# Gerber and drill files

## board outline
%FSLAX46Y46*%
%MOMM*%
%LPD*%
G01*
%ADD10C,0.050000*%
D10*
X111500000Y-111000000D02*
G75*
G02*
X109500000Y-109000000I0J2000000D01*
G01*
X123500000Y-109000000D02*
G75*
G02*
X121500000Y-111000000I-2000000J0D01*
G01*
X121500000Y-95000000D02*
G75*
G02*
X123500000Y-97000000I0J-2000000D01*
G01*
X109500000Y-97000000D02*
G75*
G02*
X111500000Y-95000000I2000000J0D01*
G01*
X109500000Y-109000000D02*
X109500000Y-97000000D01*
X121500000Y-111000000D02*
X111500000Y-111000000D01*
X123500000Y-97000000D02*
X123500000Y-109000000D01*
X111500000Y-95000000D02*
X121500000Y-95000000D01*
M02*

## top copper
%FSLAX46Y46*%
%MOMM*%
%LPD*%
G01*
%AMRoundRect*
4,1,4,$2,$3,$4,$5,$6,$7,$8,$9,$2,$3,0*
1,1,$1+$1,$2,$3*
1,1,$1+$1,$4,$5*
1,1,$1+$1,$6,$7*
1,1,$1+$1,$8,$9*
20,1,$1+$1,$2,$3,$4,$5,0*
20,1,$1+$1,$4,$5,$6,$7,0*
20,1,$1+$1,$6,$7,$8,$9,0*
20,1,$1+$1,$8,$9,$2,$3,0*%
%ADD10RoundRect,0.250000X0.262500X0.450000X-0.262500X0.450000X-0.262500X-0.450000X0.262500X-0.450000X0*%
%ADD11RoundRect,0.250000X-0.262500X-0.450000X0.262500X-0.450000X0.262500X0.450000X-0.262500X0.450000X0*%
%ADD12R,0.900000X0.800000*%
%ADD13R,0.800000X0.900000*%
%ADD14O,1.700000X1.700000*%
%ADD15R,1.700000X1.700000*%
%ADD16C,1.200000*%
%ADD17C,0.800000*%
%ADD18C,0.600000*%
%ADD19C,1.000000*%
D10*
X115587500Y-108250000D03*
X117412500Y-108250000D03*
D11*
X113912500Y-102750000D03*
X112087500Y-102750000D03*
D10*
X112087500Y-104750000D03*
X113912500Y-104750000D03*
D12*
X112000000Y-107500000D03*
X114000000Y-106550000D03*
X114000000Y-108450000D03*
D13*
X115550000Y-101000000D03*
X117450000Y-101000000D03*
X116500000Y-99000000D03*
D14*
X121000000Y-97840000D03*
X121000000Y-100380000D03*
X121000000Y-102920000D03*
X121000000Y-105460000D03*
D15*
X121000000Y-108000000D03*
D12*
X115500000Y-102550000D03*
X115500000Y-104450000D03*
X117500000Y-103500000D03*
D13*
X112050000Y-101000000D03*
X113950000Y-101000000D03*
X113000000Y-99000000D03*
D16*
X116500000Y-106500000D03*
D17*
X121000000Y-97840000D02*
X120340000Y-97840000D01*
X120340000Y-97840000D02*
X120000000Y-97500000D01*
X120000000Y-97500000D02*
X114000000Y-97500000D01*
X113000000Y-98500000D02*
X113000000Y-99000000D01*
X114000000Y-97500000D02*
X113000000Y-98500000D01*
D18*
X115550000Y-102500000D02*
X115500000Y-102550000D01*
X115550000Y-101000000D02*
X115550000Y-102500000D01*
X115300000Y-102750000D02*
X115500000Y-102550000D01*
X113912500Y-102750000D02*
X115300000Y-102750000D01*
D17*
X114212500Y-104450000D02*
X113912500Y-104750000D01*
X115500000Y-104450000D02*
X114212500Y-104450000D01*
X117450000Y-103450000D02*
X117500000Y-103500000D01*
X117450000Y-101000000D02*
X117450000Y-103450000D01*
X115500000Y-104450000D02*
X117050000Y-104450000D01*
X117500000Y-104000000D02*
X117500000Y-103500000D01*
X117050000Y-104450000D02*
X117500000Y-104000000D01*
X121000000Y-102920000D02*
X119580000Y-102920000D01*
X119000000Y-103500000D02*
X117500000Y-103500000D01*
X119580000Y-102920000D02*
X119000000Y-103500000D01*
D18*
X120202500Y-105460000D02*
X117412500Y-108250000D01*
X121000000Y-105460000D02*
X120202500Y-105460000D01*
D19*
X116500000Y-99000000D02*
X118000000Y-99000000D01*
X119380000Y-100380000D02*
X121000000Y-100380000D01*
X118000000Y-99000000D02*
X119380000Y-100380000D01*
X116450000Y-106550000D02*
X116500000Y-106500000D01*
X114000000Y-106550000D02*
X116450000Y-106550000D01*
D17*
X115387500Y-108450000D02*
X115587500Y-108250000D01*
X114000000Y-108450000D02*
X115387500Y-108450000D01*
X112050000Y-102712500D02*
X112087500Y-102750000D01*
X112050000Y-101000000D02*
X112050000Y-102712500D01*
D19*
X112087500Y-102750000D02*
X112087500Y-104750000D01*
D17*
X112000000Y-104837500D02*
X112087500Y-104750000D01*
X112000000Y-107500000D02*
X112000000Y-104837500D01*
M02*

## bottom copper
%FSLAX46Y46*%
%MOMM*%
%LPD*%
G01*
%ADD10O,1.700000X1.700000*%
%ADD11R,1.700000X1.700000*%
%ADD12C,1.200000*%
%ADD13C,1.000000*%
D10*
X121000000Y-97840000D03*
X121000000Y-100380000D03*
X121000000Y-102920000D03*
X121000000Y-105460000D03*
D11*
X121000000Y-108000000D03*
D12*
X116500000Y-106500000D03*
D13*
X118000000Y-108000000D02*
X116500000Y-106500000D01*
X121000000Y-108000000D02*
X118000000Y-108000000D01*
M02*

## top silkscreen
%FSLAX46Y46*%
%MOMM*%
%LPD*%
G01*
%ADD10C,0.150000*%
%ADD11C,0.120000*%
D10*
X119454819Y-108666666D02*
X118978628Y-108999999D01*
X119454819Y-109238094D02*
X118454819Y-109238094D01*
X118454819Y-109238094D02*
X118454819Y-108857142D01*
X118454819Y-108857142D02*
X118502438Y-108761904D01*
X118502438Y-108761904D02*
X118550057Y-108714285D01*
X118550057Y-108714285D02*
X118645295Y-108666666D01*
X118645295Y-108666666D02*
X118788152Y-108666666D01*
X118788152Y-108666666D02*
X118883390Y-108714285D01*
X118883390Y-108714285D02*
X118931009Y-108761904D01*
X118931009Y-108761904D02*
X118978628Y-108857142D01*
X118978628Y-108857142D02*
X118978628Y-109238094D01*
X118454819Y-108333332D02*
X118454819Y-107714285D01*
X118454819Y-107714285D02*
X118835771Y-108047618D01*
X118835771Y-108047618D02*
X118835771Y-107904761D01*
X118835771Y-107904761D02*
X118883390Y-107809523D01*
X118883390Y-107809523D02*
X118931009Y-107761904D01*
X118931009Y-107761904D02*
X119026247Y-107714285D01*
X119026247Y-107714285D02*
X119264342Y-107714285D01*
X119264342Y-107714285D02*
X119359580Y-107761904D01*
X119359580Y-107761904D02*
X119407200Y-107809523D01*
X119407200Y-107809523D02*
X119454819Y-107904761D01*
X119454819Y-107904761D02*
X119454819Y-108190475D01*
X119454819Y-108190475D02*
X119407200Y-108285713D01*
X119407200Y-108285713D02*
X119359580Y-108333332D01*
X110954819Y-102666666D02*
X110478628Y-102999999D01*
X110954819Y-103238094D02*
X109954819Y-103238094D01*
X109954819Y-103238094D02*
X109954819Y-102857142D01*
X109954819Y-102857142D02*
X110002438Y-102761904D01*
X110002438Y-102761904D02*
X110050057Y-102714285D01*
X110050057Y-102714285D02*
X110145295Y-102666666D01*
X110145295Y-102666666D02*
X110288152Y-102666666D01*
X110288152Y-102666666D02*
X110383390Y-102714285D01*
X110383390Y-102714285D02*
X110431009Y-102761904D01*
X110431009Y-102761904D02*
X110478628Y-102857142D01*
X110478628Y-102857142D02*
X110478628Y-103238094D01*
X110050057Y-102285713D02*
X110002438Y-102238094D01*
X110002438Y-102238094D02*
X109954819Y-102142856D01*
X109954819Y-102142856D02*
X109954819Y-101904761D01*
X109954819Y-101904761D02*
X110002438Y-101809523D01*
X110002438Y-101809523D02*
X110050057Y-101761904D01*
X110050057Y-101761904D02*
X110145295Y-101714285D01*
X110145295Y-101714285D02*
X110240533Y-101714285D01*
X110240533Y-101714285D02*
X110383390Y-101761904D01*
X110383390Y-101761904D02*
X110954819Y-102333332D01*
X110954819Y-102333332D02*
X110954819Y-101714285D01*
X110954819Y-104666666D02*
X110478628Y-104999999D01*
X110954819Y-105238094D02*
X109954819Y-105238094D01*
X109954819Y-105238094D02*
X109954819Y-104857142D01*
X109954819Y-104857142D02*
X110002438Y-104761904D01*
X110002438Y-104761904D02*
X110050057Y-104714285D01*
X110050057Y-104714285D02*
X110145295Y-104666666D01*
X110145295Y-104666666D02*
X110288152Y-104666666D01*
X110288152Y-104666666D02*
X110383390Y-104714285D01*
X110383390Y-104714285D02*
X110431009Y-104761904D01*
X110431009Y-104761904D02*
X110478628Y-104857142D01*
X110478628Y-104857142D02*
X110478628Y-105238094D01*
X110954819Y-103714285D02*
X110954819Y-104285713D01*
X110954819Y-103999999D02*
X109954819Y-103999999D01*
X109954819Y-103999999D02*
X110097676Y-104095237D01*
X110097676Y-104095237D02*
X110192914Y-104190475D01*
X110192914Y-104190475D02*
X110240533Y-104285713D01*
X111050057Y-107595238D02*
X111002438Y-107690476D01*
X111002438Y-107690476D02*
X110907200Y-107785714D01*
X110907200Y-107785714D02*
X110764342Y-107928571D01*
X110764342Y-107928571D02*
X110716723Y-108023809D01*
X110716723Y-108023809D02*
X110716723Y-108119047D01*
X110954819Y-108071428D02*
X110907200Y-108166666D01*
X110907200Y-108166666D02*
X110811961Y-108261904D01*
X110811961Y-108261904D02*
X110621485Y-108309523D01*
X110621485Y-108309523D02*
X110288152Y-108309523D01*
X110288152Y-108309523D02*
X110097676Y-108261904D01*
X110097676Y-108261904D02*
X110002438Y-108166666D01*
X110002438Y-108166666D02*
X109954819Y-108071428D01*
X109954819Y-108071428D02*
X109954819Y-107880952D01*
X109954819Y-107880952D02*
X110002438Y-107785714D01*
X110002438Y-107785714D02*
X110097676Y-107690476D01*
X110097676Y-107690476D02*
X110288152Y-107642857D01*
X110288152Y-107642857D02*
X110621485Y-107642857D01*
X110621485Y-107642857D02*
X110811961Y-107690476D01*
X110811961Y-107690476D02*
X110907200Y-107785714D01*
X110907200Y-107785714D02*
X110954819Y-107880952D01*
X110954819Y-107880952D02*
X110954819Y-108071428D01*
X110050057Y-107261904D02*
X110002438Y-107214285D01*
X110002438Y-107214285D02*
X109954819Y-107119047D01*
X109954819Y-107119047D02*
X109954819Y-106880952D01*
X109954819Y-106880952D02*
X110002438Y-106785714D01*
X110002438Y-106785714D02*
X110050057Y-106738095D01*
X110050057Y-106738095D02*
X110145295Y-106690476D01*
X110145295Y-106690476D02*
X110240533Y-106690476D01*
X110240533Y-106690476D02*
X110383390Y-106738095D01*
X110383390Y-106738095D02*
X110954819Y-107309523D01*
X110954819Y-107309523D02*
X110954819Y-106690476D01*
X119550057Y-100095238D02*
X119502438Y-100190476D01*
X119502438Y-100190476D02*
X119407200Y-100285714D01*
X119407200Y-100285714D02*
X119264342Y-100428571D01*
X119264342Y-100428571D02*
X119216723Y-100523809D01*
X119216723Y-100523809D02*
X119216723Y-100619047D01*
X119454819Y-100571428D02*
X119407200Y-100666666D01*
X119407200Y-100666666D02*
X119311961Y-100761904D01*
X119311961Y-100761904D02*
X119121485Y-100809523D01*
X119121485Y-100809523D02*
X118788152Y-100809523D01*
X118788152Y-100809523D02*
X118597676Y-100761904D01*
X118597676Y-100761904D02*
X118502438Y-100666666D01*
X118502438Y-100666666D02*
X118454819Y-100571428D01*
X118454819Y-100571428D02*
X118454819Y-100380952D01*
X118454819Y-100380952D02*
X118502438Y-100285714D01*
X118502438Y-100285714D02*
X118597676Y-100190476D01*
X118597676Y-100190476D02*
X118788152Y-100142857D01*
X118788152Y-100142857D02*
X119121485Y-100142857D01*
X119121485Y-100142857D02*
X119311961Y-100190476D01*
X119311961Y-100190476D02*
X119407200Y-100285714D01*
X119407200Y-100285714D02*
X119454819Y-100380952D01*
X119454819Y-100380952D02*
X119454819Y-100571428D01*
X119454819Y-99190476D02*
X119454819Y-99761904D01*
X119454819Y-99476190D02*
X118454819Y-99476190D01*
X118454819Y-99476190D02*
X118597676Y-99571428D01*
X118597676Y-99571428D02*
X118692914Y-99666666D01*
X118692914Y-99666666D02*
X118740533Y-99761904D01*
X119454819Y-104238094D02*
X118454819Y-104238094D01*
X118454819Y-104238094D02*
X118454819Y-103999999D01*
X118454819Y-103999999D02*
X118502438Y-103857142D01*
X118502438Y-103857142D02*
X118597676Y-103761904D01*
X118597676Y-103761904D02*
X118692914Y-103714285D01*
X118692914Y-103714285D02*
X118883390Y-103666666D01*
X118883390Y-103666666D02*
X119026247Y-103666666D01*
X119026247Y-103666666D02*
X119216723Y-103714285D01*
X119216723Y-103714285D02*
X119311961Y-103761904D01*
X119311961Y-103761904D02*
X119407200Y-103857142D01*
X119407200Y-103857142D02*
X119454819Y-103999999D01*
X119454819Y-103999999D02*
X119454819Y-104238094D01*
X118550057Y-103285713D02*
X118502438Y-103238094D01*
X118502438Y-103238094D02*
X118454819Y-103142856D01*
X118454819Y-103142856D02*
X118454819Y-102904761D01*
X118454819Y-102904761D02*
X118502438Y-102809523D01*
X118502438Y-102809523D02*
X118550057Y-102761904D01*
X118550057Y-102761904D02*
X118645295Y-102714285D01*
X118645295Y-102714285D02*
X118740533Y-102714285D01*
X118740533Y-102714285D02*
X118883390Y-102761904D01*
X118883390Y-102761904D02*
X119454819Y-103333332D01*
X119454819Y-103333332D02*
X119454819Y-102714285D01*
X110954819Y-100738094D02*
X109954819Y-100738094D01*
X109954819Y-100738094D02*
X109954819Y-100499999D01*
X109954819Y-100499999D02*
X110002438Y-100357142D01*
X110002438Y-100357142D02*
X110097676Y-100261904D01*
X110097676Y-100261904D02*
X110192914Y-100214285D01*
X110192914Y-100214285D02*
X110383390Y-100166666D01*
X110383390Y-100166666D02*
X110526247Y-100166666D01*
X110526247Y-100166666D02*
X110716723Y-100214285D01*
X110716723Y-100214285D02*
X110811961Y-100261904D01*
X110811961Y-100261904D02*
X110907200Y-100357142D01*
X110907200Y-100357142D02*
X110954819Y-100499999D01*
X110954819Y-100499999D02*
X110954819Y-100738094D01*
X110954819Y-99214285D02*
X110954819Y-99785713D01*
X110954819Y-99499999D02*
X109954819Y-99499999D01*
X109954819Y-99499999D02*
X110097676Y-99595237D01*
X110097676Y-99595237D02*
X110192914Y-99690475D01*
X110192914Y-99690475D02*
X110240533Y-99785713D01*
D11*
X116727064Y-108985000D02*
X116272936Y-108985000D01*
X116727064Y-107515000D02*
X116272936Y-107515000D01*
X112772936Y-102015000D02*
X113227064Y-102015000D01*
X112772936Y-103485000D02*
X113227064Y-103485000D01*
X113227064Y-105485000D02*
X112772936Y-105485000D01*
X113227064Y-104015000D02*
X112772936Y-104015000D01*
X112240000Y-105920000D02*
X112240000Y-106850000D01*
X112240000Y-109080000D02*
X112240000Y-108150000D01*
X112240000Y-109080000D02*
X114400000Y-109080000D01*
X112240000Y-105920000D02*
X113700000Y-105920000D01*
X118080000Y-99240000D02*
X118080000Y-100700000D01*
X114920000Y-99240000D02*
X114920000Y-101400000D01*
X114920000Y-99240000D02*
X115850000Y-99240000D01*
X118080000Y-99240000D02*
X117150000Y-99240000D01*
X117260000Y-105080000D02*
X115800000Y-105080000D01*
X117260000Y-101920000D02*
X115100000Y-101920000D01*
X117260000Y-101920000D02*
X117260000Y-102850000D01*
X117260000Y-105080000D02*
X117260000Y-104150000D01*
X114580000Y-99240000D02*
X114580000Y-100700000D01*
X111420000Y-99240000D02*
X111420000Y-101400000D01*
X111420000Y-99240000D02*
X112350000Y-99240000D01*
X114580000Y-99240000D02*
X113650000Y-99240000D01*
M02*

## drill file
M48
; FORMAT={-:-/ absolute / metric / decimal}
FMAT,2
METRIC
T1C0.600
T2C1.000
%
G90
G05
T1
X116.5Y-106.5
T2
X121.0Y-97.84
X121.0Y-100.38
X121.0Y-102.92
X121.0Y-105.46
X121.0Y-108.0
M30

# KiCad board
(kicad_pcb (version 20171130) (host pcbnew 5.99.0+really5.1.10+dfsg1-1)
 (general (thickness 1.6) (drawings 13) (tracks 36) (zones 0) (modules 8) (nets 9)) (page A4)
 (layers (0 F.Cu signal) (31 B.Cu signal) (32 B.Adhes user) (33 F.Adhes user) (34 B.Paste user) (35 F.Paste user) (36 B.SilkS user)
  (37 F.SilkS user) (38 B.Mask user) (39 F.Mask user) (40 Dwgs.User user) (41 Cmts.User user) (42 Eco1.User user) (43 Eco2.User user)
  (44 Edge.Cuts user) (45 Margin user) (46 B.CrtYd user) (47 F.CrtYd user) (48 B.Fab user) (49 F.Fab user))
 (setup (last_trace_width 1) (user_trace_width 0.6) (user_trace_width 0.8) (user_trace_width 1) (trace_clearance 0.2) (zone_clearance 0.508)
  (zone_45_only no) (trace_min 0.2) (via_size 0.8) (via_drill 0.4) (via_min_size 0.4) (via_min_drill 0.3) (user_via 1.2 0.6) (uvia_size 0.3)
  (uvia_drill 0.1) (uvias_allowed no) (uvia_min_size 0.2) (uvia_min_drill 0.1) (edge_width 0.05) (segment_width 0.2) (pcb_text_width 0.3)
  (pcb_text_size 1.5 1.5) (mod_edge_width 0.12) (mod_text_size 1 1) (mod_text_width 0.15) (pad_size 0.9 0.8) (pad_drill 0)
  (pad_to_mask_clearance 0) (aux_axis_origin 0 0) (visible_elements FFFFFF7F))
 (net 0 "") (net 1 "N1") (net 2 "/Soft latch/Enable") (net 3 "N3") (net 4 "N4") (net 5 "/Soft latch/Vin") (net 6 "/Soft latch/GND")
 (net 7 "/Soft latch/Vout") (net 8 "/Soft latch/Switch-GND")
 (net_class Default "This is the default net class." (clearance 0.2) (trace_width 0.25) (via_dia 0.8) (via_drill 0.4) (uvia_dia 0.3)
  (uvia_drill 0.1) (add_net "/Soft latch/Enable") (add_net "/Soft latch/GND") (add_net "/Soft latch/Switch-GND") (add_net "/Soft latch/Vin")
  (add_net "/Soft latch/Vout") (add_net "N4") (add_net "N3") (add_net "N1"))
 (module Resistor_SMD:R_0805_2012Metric (layer F.Cu) (at 116.5 108.25 180)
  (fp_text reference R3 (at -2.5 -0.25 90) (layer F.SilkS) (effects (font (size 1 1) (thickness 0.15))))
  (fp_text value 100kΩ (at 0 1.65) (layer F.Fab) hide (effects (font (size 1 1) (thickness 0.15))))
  (fp_line (start -0.227064 -0.735) (end 0.227064 -0.735) (layer F.SilkS) (width 0.12))
  (fp_line (start -0.227064 0.735) (end 0.227064 0.735) (layer F.SilkS) (width 0.12))
  (pad 2 smd roundrect (at 0.9125 0 180) (size 1.025 1.4) (layers F.Cu F.Paste F.Mask) (roundrect_rratio 0.243902) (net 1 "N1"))
  (pad 1 smd roundrect (at -0.9125 0 180) (size 1.025 1.4) (layers F.Cu F.Paste F.Mask) (roundrect_rratio 0.243902)
   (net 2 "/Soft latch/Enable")))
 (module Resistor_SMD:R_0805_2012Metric (layer F.Cu) (at 113 102.75)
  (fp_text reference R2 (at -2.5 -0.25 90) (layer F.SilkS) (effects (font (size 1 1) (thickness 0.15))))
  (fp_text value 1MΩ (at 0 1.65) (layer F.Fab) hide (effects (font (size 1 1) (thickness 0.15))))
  (fp_line (start -0.227064 -0.735) (end 0.227064 -0.735) (layer F.SilkS) (width 0.12))
  (fp_line (start -0.227064 0.735) (end 0.227064 0.735) (layer F.SilkS) (width 0.12))
  (pad 2 smd roundrect (at 0.9125 0) (size 1.025 1.4) (layers F.Cu F.Paste F.Mask) (roundrect_rratio 0.243902) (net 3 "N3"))
  (pad 1 smd roundrect (at -0.9125 0) (size 1.025 1.4) (layers F.Cu F.Paste F.Mask) (roundrect_rratio 0.243902) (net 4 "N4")))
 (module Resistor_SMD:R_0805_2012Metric (layer F.Cu) (at 113 104.75 180)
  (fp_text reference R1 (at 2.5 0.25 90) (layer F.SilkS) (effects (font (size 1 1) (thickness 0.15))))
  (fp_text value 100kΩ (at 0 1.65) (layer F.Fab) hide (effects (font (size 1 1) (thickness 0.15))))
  (fp_line (start -0.227064 -0.735) (end 0.227064 -0.735) (layer F.SilkS) (width 0.12))
  (fp_line (start -0.227064 0.735) (end 0.227064 0.735) (layer F.SilkS) (width 0.12))
  (pad 2 smd roundrect (at 0.9125 0 180) (size 1.025 1.4) (layers F.Cu F.Paste F.Mask) (roundrect_rratio 0.243902) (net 4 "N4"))
  (pad 1 smd roundrect (at -0.9125 0 180) (size 1.025 1.4) (layers F.Cu F.Paste F.Mask) (roundrect_rratio 0.243902)
   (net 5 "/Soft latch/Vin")))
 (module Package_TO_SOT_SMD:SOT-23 (layer F.Cu) (at 113 107.5 180)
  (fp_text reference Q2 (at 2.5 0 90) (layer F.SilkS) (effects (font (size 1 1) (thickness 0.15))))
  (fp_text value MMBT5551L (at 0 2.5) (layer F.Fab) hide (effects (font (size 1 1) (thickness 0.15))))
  (fp_line (start 0.76 1.58) (end 0.76 0.65) (layer F.SilkS) (width 0.12))
  (fp_line (start 0.76 -1.58) (end 0.76 -0.65) (layer F.SilkS) (width 0.12))
  (fp_line (start 0.76 -1.58) (end -1.4 -1.58) (layer F.SilkS) (width 0.12))
  (fp_line (start 0.76 1.58) (end -0.7 1.58) (layer F.SilkS) (width 0.12))
  (pad 3 smd rect (at 1 0 180) (size 0.9 0.8) (layers F.Cu F.Paste F.Mask) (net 4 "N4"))
  (pad 2 smd rect (at -1 0.95 180) (size 0.9 0.8) (layers F.Cu F.Paste F.Mask) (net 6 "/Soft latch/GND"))
  (pad 1 smd rect (at -1 -0.95 180) (size 0.9 0.8) (layers F.Cu F.Paste F.Mask) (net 1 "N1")))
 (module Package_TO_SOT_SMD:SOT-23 (layer F.Cu) (at 116.5 100 90)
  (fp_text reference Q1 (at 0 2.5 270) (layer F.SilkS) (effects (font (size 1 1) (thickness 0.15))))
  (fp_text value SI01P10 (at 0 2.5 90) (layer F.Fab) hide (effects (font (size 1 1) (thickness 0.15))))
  (fp_line (start 0.76 1.58) (end -0.7 1.58) (layer F.SilkS) (width 0.12))
  (fp_line (start 0.76 -1.58) (end -1.4 -1.58) (layer F.SilkS) (width 0.12))
  (fp_line (start 0.76 -1.58) (end 0.76 -0.65) (layer F.SilkS) (width 0.12))
  (fp_line (start 0.76 1.58) (end 0.76 0.65) (layer F.SilkS) (width 0.12))
  (pad 1 smd rect (at -1 -0.95 90) (size 0.9 0.8) (layers F.Cu F.Paste F.Mask) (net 3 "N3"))
  (pad 2 smd rect (at -1 0.95 90) (size 0.9 0.8) (layers F.Cu F.Paste F.Mask) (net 5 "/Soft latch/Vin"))
  (pad 3 smd rect (at 1 0 90) (size 0.9 0.8) (layers F.Cu F.Paste F.Mask) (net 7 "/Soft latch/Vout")))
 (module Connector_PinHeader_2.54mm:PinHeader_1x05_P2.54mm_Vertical (layer B.Cu) (at 121 108)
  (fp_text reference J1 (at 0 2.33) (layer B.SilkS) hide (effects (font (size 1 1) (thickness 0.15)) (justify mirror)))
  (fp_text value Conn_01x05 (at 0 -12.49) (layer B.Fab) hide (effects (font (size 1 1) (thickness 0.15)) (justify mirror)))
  (pad 5 thru_hole oval (at 0 -10.16) (size 1.7 1.7) (drill 1) (layers *.Cu *.Mask) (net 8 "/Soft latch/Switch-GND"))
  (pad 4 thru_hole oval (at 0 -7.62) (size 1.7 1.7) (drill 1) (layers *.Cu *.Mask) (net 7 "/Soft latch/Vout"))
  (pad 3 thru_hole oval (at 0 -5.08) (size 1.7 1.7) (drill 1) (layers *.Cu *.Mask) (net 5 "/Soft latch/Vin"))
  (pad 2 thru_hole oval (at 0 -2.54) (size 1.7 1.7) (drill 1) (layers *.Cu *.Mask) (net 2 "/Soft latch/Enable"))
  (pad 1 thru_hole rect (at 0 0) (size 1.7 1.7) (drill 1) (layers *.Cu *.Mask) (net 6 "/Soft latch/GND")))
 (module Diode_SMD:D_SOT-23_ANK (layer F.Cu) (at 116.5 103.5)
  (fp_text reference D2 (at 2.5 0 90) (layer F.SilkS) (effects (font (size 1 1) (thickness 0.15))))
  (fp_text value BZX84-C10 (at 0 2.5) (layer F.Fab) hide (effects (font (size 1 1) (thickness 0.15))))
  (fp_line (start 0.76 1.58) (end -0.7 1.58) (layer F.SilkS) (width 0.12))
  (fp_line (start 0.76 -1.58) (end -1.4 -1.58) (layer F.SilkS) (width 0.12))
  (fp_line (start 0.76 -1.58) (end 0.76 -0.65) (layer F.SilkS) (width 0.12))
  (fp_line (start 0.76 1.58) (end 0.76 0.65) (layer F.SilkS) (width 0.12))
  (pad 2 smd rect (at -1 -0.95) (size 0.9 0.8) (layers F.Cu F.Paste F.Mask) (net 3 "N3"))
  (pad "" smd rect (at -1 0.95) (size 0.9 0.8) (layers F.Cu F.Paste F.Mask) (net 5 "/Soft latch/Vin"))
  (pad 1 smd rect (at 1 0) (size 0.9 0.8) (layers F.Cu F.Paste F.Mask) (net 5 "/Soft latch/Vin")))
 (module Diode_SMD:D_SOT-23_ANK (layer F.Cu) (at 113 100 90)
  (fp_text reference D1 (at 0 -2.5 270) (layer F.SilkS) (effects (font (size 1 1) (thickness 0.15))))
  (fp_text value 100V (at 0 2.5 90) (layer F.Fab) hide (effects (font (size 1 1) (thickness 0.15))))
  (fp_line (start 0.76 1.58) (end -0.7 1.58) (layer F.SilkS) (width 0.12))
  (fp_line (start 0.76 -1.58) (end -1.4 -1.58) (layer F.SilkS) (width 0.12))
  (fp_line (start 0.76 -1.58) (end 0.76 -0.65) (layer F.SilkS) (width 0.12))
  (fp_line (start 0.76 1.58) (end 0.76 0.65) (layer F.SilkS) (width 0.12))
  (pad 2 smd rect (at -1 -0.95 90) (size 0.9 0.8) (layers F.Cu F.Paste F.Mask) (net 4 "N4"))
  (pad "" smd rect (at -1 0.95 90) (size 0.9 0.8) (layers F.Cu F.Paste F.Mask))
  (pad 1 smd rect (at 1 0 90) (size 0.9 0.8) (layers F.Cu F.Paste F.Mask) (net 8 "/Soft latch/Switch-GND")))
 (gr_arc (start 111.5 109) (end 109.5 109) (angle -90) (layer Edge.Cuts) (width 0.05))
 (gr_arc (start 121.5 109) (end 121.5 111) (angle -90) (layer Edge.Cuts) (width 0.05))
 (gr_arc (start 121.5 97) (end 123.5 97) (angle -90) (layer Edge.Cuts) (width 0.05))
 (gr_arc (start 111.5 97) (end 111.5 95) (angle -90) (layer Edge.Cuts) (width 0.05))
 (gr_line (start 109.5 109) (end 109.5 97) (layer Edge.Cuts) (width 0.05))
 (gr_line (start 121.5 111) (end 111.5 111) (layer Edge.Cuts) (width 0.05))
 (gr_line (start 123.5 97) (end 123.5 109) (layer Edge.Cuts) (width 0.05))
 (gr_line (start 111.5 95) (end 121.5 95) (layer Edge.Cuts) (width 0.05))
 (via (at 116.5 106.5) (size 1.2) (drill 0.6) (layers F.Cu B.Cu) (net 6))
 (segment (start 121 97.84) (end 120.34 97.84) (width 0.8) (layer F.Cu) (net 8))
 (segment (start 120.34 97.84) (end 120 97.5) (width 0.8) (layer F.Cu) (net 8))
 (segment (start 120 97.5) (end 114 97.5) (width 0.8) (layer F.Cu) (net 8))
 (segment (start 113 98.5) (end 113 99) (width 0.8) (layer F.Cu) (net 8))
 (segment (start 114 97.5) (end 113 98.5) (width 0.8) (layer F.Cu) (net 8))
 (segment (start 115.55 102.5) (end 115.5 102.55) (width 0.6) (layer F.Cu) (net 3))
 (segment (start 115.55 101) (end 115.55 102.5) (width 0.6) (layer F.Cu) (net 3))
 (segment (start 115.3 102.75) (end 115.5 102.55) (width 0.6) (layer F.Cu) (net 3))
 (segment (start 113.9125 102.75) (end 115.3 102.75) (width 0.6) (layer F.Cu) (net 3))
 (segment (start 114.2125 104.45) (end 113.9125 104.75) (width 0.8) (layer F.Cu) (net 5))
 (segment (start 115.5 104.45) (end 114.2125 104.45) (width 0.8) (layer F.Cu) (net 5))
 (segment (start 117.45 103.45) (end 117.5 103.5) (width 0.8) (layer F.Cu) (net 5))
 (segment (start 117.45 101) (end 117.45 103.45) (width 0.8) (layer F.Cu) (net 5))
 (segment (start 115.5 104.45) (end 117.05 104.45) (width 0.8) (layer F.Cu) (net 5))
 (segment (start 117.5 104) (end 117.5 103.5) (width 0.8) (layer F.Cu) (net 5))
 (segment (start 117.05 104.45) (end 117.5 104) (width 0.8) (layer F.Cu) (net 5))
 (segment (start 121 102.92) (end 119.58 102.92) (width 0.8) (layer F.Cu) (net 5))
 (segment (start 119 103.5) (end 117.5 103.5) (width 0.8) (layer F.Cu) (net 5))
 (segment (start 119.58 102.92) (end 119 103.5) (width 0.8) (layer F.Cu) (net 5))
 (segment (start 120.2025 105.46) (end 117.4125 108.25) (width 0.6) (layer F.Cu) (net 2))
 (segment (start 121 105.46) (end 120.2025 105.46) (width 0.6) (layer F.Cu) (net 2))
 (segment (start 116.5 99) (end 118 99) (width 1) (layer F.Cu) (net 7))
 (segment (start 119.38 100.38) (end 121 100.38) (width 1) (layer F.Cu) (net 7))
 (segment (start 118 99) (end 119.38 100.38) (width 1) (layer F.Cu) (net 7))
 (segment (start 116.45 106.55) (end 116.5 106.5) (width 1) (layer F.Cu) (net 6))
 (segment (start 114 106.55) (end 116.45 106.55) (width 1) (layer F.Cu) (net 6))
 (segment (start 118 108) (end 116.5 106.5) (width 1) (layer B.Cu) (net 6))
 (segment (start 121 108) (end 118 108) (width 1) (layer B.Cu) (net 6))
 (segment (start 115.3875 108.45) (end 115.5875 108.25) (width 0.8) (layer F.Cu) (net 1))
 (segment (start 114 108.45) (end 115.3875 108.45) (width 0.8) (layer F.Cu) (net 1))
 (segment (start 112.05 102.7125) (end 112.0875 102.75) (width 0.8) (layer F.Cu) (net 4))
 (segment (start 112.05 101) (end 112.05 102.7125) (width 0.8) (layer F.Cu) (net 4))
 (segment (start 112.0875 102.75) (end 112.0875 104.75) (width 1) (layer F.Cu) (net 4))
 (segment (start 112 104.8375) (end 112.0875 104.75) (width 0.8) (layer F.Cu) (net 4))
 (segment (start 112 107.5) (end 112 104.8375) (width 0.8) (layer F.Cu) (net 4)))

